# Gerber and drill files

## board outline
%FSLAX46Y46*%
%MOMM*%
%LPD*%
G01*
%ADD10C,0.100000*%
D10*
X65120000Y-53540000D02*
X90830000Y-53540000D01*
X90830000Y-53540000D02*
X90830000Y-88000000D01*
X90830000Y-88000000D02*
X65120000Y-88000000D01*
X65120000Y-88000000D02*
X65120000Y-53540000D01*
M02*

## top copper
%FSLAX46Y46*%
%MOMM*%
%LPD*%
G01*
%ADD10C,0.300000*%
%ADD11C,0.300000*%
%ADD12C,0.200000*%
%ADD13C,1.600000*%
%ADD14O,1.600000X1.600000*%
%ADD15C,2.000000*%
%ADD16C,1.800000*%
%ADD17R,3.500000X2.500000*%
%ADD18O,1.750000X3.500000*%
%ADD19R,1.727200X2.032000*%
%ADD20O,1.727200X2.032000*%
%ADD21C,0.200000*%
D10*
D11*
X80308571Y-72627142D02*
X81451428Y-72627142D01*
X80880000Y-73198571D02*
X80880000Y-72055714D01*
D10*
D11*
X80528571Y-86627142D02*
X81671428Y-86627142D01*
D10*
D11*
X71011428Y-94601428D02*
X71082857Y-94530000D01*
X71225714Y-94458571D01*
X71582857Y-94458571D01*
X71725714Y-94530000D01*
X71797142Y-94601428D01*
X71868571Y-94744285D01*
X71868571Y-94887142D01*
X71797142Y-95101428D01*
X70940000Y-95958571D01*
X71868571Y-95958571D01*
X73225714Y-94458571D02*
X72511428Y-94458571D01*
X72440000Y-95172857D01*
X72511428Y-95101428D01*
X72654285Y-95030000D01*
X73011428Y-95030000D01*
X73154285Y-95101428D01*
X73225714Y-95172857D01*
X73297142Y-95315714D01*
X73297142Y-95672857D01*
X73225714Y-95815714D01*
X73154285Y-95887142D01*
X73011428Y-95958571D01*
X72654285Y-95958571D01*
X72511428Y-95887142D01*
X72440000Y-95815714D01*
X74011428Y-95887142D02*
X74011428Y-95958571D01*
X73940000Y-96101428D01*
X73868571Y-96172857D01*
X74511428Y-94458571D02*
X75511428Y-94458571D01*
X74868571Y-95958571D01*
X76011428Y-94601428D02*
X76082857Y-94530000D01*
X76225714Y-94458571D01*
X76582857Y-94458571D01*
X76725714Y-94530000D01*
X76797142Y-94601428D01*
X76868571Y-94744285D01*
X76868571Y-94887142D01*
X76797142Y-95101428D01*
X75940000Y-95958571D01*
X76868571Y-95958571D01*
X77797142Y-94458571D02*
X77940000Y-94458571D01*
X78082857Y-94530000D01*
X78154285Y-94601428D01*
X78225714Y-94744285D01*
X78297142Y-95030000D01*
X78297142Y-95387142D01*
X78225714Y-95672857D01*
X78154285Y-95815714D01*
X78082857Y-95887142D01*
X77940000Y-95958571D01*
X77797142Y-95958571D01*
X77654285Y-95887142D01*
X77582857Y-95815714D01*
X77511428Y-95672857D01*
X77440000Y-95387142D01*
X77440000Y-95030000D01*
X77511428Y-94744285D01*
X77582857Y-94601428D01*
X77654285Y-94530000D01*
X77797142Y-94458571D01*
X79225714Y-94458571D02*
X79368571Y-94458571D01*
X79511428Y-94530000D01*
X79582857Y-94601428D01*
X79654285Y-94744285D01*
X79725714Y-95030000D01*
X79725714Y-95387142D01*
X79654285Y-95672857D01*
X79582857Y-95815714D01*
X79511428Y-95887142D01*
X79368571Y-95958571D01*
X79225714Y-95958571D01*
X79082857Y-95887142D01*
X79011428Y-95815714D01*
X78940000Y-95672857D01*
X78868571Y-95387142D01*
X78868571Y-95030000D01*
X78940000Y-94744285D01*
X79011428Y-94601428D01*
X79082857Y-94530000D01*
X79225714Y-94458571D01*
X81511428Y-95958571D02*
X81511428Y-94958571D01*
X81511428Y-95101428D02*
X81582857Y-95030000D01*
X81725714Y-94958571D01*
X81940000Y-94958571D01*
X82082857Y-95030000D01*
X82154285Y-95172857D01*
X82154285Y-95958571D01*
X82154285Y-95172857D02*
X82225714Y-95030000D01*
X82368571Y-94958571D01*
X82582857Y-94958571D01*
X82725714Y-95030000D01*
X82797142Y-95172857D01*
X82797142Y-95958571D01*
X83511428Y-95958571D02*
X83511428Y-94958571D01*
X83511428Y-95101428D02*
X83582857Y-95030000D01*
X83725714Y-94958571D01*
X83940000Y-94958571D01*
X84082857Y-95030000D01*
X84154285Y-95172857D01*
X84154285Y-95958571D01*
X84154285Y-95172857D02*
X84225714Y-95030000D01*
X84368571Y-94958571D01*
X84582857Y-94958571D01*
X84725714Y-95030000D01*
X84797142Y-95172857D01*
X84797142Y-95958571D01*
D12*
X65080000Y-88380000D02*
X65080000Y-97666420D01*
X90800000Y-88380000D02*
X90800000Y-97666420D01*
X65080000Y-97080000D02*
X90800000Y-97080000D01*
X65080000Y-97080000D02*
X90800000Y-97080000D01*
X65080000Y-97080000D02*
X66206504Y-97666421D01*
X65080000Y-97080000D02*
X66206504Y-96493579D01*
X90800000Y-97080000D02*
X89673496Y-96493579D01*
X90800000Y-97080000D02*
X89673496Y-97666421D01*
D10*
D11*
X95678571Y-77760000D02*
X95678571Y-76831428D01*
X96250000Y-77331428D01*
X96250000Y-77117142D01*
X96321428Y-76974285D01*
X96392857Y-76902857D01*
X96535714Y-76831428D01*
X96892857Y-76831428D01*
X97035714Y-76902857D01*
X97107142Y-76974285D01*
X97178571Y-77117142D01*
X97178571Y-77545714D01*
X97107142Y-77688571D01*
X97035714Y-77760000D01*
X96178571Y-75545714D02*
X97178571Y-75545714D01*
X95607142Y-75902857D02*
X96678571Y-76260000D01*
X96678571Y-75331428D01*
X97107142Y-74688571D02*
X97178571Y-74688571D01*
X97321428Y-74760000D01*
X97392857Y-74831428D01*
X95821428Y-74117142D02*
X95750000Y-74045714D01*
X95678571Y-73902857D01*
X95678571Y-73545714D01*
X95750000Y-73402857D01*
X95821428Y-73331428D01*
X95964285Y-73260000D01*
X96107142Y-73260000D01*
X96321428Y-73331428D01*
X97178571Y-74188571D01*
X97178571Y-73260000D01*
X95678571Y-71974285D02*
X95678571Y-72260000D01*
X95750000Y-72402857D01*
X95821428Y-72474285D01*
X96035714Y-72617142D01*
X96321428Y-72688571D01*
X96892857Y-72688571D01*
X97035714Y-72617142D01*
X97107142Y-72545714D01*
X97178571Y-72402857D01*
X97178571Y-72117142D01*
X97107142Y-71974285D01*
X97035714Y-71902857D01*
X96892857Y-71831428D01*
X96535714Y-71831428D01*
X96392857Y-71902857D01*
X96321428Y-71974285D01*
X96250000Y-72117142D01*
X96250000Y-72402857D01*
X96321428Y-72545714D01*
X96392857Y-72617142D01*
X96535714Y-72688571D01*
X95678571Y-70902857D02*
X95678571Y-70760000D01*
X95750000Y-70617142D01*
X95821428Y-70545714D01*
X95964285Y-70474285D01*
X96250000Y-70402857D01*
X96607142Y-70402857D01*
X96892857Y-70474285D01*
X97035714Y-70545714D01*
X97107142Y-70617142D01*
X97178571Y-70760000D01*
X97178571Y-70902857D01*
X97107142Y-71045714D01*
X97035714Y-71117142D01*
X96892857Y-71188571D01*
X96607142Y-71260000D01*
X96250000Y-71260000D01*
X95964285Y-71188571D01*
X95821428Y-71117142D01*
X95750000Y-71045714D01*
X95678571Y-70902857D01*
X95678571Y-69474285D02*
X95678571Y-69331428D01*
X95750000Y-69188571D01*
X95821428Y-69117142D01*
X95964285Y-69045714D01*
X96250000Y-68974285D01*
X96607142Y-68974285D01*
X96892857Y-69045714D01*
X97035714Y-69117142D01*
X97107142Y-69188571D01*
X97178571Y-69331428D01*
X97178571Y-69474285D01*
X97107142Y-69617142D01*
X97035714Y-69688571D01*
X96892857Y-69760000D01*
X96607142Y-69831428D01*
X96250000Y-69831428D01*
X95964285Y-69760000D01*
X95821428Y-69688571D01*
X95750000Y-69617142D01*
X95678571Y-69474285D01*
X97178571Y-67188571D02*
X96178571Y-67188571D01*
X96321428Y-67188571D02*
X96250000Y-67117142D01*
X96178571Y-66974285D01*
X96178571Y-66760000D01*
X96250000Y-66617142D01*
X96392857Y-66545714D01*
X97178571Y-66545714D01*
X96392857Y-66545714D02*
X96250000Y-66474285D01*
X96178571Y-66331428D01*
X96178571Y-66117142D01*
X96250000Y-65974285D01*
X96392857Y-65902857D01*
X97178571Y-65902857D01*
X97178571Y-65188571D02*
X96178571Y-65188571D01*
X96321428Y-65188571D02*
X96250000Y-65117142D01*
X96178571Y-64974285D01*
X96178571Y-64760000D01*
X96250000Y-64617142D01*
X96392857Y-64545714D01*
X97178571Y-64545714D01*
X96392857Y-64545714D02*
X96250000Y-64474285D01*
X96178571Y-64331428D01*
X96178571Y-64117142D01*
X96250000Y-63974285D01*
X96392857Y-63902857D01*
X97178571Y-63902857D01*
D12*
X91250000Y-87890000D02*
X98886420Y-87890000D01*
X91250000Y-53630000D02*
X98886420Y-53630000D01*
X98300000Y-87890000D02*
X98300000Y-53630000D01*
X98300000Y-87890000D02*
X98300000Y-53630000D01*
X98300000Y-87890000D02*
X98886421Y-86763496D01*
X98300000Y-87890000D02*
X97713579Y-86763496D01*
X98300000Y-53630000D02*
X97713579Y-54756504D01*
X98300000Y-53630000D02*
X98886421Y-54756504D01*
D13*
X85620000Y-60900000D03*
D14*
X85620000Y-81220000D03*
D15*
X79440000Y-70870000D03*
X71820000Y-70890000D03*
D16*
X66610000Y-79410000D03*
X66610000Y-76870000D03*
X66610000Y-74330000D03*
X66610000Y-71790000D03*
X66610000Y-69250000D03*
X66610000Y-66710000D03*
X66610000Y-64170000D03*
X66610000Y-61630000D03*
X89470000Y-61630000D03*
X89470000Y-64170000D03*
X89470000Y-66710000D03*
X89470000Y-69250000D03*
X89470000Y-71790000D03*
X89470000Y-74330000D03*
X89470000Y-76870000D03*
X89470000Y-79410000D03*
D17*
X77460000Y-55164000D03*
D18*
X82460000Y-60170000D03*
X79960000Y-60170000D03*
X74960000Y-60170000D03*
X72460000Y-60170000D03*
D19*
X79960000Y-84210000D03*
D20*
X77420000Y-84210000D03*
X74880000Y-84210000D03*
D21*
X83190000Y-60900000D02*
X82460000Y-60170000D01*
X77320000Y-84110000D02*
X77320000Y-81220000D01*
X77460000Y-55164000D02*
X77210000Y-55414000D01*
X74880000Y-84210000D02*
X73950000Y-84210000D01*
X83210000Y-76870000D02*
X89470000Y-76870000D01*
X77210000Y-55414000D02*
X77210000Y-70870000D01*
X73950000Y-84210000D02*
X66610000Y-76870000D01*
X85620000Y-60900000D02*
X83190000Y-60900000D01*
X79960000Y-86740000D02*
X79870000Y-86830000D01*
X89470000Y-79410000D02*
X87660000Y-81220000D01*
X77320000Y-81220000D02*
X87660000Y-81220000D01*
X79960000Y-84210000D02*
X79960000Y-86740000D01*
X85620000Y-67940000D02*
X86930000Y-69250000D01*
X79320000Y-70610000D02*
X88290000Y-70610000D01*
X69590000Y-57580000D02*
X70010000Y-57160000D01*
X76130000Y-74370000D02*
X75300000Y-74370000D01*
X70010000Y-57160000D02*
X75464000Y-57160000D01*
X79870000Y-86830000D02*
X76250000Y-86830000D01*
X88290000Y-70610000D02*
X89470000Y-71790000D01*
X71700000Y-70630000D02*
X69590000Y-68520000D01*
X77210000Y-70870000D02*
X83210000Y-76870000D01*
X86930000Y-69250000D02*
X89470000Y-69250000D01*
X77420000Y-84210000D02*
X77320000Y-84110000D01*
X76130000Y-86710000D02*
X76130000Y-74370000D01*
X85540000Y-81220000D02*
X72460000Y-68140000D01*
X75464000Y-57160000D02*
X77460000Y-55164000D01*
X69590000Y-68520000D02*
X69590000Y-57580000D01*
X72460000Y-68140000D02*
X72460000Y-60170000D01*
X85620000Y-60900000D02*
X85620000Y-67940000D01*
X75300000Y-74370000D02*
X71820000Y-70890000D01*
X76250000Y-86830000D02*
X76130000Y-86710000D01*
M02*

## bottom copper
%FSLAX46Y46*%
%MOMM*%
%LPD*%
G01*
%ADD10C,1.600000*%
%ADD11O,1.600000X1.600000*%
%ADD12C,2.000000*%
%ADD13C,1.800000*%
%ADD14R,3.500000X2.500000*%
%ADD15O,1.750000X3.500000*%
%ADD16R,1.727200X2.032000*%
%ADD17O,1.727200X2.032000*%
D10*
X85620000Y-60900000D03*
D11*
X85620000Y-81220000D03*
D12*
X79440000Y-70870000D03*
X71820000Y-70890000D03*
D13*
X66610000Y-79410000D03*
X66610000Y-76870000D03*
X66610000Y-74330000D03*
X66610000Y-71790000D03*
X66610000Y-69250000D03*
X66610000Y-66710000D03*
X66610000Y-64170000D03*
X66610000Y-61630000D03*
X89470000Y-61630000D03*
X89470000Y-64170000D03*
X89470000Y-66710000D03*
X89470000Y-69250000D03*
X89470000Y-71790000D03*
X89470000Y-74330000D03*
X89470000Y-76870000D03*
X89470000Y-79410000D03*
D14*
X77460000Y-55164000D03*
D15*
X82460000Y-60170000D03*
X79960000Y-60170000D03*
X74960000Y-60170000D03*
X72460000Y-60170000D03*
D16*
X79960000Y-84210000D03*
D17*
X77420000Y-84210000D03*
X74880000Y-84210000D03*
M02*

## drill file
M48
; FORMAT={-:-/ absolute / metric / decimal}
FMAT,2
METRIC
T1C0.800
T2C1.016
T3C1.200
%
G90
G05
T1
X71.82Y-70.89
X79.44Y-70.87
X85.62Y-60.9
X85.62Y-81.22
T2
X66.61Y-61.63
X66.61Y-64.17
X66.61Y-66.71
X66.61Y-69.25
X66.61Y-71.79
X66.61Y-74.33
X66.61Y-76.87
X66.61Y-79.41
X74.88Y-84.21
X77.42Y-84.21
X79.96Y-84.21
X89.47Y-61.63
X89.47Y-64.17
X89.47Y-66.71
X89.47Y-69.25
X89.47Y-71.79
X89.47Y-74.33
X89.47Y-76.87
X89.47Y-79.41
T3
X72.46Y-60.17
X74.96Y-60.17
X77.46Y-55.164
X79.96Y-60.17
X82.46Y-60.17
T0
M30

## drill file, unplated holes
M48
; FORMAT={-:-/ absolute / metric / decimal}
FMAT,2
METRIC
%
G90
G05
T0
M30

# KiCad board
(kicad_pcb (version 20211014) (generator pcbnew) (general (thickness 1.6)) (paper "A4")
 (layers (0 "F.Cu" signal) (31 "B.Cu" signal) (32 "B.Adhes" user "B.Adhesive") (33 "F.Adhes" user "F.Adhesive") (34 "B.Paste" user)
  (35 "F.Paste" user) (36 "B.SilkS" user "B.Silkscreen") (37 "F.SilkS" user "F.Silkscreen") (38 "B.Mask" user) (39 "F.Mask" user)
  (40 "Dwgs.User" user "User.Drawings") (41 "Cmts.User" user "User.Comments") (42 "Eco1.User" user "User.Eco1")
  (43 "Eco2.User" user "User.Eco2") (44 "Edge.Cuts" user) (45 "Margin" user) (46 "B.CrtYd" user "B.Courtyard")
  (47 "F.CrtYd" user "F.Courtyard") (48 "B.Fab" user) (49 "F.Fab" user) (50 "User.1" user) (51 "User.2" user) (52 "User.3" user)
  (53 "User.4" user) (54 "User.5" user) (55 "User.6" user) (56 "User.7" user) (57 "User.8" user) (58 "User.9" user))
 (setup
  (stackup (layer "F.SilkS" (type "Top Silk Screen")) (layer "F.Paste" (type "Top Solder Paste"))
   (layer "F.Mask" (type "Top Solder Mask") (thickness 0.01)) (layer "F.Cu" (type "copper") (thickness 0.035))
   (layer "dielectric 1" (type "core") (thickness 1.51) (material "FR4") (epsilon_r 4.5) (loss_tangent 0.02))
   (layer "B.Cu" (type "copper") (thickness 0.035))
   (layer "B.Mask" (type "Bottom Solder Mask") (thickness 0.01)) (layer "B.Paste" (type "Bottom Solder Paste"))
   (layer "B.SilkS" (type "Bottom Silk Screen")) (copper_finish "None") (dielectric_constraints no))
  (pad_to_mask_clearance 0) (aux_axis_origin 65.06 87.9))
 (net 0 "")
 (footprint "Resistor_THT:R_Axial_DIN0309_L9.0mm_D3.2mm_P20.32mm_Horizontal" (layer "F.Cu") (at 85.62 60.9 -90)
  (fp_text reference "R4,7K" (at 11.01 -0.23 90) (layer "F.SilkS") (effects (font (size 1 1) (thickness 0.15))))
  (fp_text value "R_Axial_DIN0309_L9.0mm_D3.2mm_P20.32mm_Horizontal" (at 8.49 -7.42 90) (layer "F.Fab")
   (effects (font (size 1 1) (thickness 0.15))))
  (pad "1" thru_hole circle (at 0 0 270) (size 1.6 1.6) (drill 0.8) (layers *.Cu *.Mask))
  (pad "2" thru_hole oval (at 20.32 0 270) (size 1.6 1.6) (drill 0.8) (layers *.Cu *.Mask)))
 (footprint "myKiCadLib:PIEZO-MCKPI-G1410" (layer "F.Cu") (at 75.63 70.88 180)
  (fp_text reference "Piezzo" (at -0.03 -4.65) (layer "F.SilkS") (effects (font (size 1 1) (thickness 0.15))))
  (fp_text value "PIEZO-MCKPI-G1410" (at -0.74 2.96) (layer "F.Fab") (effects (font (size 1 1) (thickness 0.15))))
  (pad "1" thru_hole circle locked (at -3.81 0.01 180) (size 2 2) (drill 0.8) (layers *.Cu *.Mask "F.SilkS"))
  (pad "2" thru_hole circle locked (at 3.81 -0.01 180) (size 2 2) (drill 0.8) (layers *.Cu *.Mask "F.SilkS")))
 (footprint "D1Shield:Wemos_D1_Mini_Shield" (layer "F.Cu") (at 78.04 71.79)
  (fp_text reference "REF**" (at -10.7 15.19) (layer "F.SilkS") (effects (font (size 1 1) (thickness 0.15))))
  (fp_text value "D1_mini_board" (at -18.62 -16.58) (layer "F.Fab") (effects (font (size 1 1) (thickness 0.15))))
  (pad "1" thru_hole circle locked (at -11.43 7.62) (size 1.8 1.8) (drill 1.016) (layers *.Cu *.Mask "F.SilkS"))
  (pad "2" thru_hole circle locked (at -11.43 5.08) (size 1.8 1.8) (drill 1.016) (layers *.Cu *.Mask "F.SilkS"))
  (pad "3" thru_hole circle locked (at -11.43 2.54) (size 1.8 1.8) (drill 1.016) (layers *.Cu *.Mask "F.SilkS"))
  (pad "4" thru_hole circle locked (at -11.43 0) (size 1.8 1.8) (drill 1.016) (layers *.Cu *.Mask "F.SilkS"))
  (pad "5" thru_hole circle locked (at -11.43 -2.54) (size 1.8 1.8) (drill 1.016) (layers *.Cu *.Mask "F.SilkS"))
  (pad "6" thru_hole circle locked (at -11.43 -5.08) (size 1.8 1.8) (drill 1.016) (layers *.Cu *.Mask "F.SilkS"))
  (pad "7" thru_hole circle locked (at -11.43 -7.62) (size 1.8 1.8) (drill 1.016) (layers *.Cu *.Mask "F.SilkS"))
  (pad "8" thru_hole circle locked (at -11.43 -10.16) (size 1.8 1.8) (drill 1.016) (layers *.Cu *.Mask "F.SilkS"))
  (pad "9" thru_hole circle locked (at 11.43 -10.16) (size 1.8 1.8) (drill 1.016) (layers *.Cu *.Mask "F.SilkS"))
  (pad "10" thru_hole circle locked (at 11.43 -7.62) (size 1.8 1.8) (drill 1.016) (layers *.Cu *.Mask "F.SilkS"))
  (pad "11" thru_hole circle locked (at 11.43 -5.08) (size 1.8 1.8) (drill 1.016) (layers *.Cu *.Mask "F.SilkS"))
  (pad "12" thru_hole circle locked (at 11.43 -2.54) (size 1.8 1.8) (drill 1.016) (layers *.Cu *.Mask "F.SilkS"))
  (pad "13" thru_hole circle locked (at 11.43 0) (size 1.8 1.8) (drill 1.016) (layers *.Cu *.Mask "F.SilkS"))
  (pad "14" thru_hole circle locked (at 11.43 2.54) (size 1.8 1.8) (drill 1.016) (layers *.Cu *.Mask "F.SilkS"))
  (pad "15" thru_hole circle locked (at 11.43 5.08) (size 1.8 1.8) (drill 1.016) (layers *.Cu *.Mask "F.SilkS"))
  (pad "16" thru_hole circle locked (at 11.43 7.62) (size 1.8 1.8) (drill 1.016) (layers *.Cu *.Mask "F.SilkS")))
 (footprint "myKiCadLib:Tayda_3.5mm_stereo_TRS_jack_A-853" (layer "F.Cu") (at 77.46 56.76)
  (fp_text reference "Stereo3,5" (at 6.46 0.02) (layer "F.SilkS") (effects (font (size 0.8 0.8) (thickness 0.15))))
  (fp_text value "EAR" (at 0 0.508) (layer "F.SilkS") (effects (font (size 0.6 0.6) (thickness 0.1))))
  (pad "1" thru_hole rect locked (at 0 -1.596) (size 3.5 2.5) (drill 1.2) (layers *.Cu *.Mask "F.SilkS"))
  (pad "2" thru_hole oval locked (at 5 3.41) (size 1.75 3.5) (drill 1.2) (layers *.Cu *.Mask "F.SilkS"))
  (pad "3" thru_hole oval locked (at 2.5 3.41) (size 1.75 3.5) (drill 1.2) (layers *.Cu *.Mask "F.SilkS"))
  (pad "4" thru_hole oval locked (at -2.5 3.41) (size 1.75 3.5) (drill 1.2) (layers *.Cu *.Mask "F.SilkS"))
  (pad "5" thru_hole oval locked (at -5 3.41) (size 1.75 3.5) (drill 1.2) (layers *.Cu *.Mask "F.SilkS")))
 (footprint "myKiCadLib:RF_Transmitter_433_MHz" (layer "F.Cu") (at 77.42 84.21 180)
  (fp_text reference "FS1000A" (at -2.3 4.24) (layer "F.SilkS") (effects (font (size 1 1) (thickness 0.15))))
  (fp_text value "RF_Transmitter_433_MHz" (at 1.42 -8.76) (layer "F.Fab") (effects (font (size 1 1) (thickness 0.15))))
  (pad "1" thru_hole rect locked (at -2.54 0 270) (size 2.032 1.7272) (drill 1.016) (layers *.Cu *.Mask "F.SilkS"))
  (pad "2" thru_hole oval locked (at 0 0 270) (size 2.032 1.7272) (drill 1.016) (layers *.Cu *.Mask "F.SilkS"))
  (pad "3" thru_hole oval locked (at 2.54 0 270) (size 2.032 1.7272) (drill 1.016) (layers *.Cu *.Mask "F.SilkS")))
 (gr_rect (start 65.12 53.54) (end 90.83 88) (layer "Edge.Cuts") (width 0.1) (fill none))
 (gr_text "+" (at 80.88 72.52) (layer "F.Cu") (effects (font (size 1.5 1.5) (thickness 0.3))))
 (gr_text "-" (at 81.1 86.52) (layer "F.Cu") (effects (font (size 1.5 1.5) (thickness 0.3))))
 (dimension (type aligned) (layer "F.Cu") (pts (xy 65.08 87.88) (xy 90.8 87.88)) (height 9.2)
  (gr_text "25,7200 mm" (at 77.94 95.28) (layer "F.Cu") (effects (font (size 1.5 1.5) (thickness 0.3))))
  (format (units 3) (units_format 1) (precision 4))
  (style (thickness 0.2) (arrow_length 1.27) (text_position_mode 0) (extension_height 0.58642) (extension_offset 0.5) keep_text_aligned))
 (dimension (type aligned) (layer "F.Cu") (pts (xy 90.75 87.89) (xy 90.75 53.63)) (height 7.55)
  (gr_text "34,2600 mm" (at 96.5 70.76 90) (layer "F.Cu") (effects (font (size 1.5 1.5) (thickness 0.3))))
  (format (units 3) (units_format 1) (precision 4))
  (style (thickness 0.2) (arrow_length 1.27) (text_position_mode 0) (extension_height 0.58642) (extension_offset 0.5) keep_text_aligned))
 (segment (start 83.19 60.9) (end 82.46 60.17) (width 0.2) (layer "F.Cu") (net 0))
 (segment (start 77.32 84.11) (end 77.32 81.22) (width 0.2) (layer "F.Cu") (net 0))
 (segment (start 77.46 55.164) (end 77.21 55.414) (width 0.2) (layer "F.Cu") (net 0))
 (segment (start 74.88 84.21) (end 73.95 84.21) (width 0.2) (layer "F.Cu") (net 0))
 (segment (start 83.21 76.87) (end 89.47 76.87) (width 0.2) (layer "F.Cu") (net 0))
 (segment (start 77.21 55.414) (end 77.21 70.87) (width 0.2) (layer "F.Cu") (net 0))
 (segment (start 73.95 84.21) (end 66.61 76.87) (width 0.2) (layer "F.Cu") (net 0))
 (segment (start 85.62 60.9) (end 83.19 60.9) (width 0.2) (layer "F.Cu") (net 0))
 (segment (start 79.96 86.74) (end 79.87 86.83) (width 0.2) (layer "F.Cu") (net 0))
 (segment (start 89.47 79.41) (end 87.66 81.22) (width 0.2) (layer "F.Cu") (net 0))
 (segment (start 77.32 81.22) (end 87.66 81.22) (width 0.2) (layer "F.Cu") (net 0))
 (segment (start 79.96 84.21) (end 79.96 86.74) (width 0.2) (layer "F.Cu") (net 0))
 (segment (start 85.62 67.94) (end 86.93 69.25) (width 0.2) (layer "F.Cu") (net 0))
 (segment (start 79.32 70.61) (end 88.29 70.61) (width 0.2) (layer "F.Cu") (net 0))
 (segment (start 69.59 57.58) (end 70.01 57.16) (width 0.2) (layer "F.Cu") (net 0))
 (segment (start 76.13 74.37) (end 75.3 74.37) (width 0.2) (layer "F.Cu") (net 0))
 (segment (start 70.01 57.16) (end 75.464 57.16) (width 0.2) (layer "F.Cu") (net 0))
 (segment (start 79.87 86.83) (end 76.25 86.83) (width 0.2) (layer "F.Cu") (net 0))
 (segment (start 88.29 70.61) (end 89.47 71.79) (width 0.2) (layer "F.Cu") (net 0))
 (segment (start 71.7 70.63) (end 69.59 68.52) (width 0.2) (layer "F.Cu") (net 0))
 (segment (start 77.21 70.87) (end 83.21 76.87) (width 0.2) (layer "F.Cu") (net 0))
 (segment (start 86.93 69.25) (end 89.47 69.25) (width 0.2) (layer "F.Cu") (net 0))
 (segment (start 77.42 84.21) (end 77.32 84.11) (width 0.2) (layer "F.Cu") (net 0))
 (segment (start 76.13 86.71) (end 76.13 74.37) (width 0.2) (layer "F.Cu") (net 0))
 (segment (start 85.54 81.22) (end 72.46 68.14) (width 0.2) (layer "F.Cu") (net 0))
 (segment (start 75.464 57.16) (end 77.46 55.164) (width 0.2) (layer "F.Cu") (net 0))
 (segment (start 69.59 68.52) (end 69.59 57.58) (width 0.2) (layer "F.Cu") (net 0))
 (segment (start 72.46 68.14) (end 72.46 60.17) (width 0.2) (layer "F.Cu") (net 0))
 (segment (start 85.62 60.9) (end 85.62 67.94) (width 0.2) (layer "F.Cu") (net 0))
 (segment (start 75.3 74.37) (end 71.82 70.89) (width 0.2) (layer "F.Cu") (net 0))
 (segment (start 76.25 86.83) (end 76.13 86.71) (width 0.2) (layer "F.Cu") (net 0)))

